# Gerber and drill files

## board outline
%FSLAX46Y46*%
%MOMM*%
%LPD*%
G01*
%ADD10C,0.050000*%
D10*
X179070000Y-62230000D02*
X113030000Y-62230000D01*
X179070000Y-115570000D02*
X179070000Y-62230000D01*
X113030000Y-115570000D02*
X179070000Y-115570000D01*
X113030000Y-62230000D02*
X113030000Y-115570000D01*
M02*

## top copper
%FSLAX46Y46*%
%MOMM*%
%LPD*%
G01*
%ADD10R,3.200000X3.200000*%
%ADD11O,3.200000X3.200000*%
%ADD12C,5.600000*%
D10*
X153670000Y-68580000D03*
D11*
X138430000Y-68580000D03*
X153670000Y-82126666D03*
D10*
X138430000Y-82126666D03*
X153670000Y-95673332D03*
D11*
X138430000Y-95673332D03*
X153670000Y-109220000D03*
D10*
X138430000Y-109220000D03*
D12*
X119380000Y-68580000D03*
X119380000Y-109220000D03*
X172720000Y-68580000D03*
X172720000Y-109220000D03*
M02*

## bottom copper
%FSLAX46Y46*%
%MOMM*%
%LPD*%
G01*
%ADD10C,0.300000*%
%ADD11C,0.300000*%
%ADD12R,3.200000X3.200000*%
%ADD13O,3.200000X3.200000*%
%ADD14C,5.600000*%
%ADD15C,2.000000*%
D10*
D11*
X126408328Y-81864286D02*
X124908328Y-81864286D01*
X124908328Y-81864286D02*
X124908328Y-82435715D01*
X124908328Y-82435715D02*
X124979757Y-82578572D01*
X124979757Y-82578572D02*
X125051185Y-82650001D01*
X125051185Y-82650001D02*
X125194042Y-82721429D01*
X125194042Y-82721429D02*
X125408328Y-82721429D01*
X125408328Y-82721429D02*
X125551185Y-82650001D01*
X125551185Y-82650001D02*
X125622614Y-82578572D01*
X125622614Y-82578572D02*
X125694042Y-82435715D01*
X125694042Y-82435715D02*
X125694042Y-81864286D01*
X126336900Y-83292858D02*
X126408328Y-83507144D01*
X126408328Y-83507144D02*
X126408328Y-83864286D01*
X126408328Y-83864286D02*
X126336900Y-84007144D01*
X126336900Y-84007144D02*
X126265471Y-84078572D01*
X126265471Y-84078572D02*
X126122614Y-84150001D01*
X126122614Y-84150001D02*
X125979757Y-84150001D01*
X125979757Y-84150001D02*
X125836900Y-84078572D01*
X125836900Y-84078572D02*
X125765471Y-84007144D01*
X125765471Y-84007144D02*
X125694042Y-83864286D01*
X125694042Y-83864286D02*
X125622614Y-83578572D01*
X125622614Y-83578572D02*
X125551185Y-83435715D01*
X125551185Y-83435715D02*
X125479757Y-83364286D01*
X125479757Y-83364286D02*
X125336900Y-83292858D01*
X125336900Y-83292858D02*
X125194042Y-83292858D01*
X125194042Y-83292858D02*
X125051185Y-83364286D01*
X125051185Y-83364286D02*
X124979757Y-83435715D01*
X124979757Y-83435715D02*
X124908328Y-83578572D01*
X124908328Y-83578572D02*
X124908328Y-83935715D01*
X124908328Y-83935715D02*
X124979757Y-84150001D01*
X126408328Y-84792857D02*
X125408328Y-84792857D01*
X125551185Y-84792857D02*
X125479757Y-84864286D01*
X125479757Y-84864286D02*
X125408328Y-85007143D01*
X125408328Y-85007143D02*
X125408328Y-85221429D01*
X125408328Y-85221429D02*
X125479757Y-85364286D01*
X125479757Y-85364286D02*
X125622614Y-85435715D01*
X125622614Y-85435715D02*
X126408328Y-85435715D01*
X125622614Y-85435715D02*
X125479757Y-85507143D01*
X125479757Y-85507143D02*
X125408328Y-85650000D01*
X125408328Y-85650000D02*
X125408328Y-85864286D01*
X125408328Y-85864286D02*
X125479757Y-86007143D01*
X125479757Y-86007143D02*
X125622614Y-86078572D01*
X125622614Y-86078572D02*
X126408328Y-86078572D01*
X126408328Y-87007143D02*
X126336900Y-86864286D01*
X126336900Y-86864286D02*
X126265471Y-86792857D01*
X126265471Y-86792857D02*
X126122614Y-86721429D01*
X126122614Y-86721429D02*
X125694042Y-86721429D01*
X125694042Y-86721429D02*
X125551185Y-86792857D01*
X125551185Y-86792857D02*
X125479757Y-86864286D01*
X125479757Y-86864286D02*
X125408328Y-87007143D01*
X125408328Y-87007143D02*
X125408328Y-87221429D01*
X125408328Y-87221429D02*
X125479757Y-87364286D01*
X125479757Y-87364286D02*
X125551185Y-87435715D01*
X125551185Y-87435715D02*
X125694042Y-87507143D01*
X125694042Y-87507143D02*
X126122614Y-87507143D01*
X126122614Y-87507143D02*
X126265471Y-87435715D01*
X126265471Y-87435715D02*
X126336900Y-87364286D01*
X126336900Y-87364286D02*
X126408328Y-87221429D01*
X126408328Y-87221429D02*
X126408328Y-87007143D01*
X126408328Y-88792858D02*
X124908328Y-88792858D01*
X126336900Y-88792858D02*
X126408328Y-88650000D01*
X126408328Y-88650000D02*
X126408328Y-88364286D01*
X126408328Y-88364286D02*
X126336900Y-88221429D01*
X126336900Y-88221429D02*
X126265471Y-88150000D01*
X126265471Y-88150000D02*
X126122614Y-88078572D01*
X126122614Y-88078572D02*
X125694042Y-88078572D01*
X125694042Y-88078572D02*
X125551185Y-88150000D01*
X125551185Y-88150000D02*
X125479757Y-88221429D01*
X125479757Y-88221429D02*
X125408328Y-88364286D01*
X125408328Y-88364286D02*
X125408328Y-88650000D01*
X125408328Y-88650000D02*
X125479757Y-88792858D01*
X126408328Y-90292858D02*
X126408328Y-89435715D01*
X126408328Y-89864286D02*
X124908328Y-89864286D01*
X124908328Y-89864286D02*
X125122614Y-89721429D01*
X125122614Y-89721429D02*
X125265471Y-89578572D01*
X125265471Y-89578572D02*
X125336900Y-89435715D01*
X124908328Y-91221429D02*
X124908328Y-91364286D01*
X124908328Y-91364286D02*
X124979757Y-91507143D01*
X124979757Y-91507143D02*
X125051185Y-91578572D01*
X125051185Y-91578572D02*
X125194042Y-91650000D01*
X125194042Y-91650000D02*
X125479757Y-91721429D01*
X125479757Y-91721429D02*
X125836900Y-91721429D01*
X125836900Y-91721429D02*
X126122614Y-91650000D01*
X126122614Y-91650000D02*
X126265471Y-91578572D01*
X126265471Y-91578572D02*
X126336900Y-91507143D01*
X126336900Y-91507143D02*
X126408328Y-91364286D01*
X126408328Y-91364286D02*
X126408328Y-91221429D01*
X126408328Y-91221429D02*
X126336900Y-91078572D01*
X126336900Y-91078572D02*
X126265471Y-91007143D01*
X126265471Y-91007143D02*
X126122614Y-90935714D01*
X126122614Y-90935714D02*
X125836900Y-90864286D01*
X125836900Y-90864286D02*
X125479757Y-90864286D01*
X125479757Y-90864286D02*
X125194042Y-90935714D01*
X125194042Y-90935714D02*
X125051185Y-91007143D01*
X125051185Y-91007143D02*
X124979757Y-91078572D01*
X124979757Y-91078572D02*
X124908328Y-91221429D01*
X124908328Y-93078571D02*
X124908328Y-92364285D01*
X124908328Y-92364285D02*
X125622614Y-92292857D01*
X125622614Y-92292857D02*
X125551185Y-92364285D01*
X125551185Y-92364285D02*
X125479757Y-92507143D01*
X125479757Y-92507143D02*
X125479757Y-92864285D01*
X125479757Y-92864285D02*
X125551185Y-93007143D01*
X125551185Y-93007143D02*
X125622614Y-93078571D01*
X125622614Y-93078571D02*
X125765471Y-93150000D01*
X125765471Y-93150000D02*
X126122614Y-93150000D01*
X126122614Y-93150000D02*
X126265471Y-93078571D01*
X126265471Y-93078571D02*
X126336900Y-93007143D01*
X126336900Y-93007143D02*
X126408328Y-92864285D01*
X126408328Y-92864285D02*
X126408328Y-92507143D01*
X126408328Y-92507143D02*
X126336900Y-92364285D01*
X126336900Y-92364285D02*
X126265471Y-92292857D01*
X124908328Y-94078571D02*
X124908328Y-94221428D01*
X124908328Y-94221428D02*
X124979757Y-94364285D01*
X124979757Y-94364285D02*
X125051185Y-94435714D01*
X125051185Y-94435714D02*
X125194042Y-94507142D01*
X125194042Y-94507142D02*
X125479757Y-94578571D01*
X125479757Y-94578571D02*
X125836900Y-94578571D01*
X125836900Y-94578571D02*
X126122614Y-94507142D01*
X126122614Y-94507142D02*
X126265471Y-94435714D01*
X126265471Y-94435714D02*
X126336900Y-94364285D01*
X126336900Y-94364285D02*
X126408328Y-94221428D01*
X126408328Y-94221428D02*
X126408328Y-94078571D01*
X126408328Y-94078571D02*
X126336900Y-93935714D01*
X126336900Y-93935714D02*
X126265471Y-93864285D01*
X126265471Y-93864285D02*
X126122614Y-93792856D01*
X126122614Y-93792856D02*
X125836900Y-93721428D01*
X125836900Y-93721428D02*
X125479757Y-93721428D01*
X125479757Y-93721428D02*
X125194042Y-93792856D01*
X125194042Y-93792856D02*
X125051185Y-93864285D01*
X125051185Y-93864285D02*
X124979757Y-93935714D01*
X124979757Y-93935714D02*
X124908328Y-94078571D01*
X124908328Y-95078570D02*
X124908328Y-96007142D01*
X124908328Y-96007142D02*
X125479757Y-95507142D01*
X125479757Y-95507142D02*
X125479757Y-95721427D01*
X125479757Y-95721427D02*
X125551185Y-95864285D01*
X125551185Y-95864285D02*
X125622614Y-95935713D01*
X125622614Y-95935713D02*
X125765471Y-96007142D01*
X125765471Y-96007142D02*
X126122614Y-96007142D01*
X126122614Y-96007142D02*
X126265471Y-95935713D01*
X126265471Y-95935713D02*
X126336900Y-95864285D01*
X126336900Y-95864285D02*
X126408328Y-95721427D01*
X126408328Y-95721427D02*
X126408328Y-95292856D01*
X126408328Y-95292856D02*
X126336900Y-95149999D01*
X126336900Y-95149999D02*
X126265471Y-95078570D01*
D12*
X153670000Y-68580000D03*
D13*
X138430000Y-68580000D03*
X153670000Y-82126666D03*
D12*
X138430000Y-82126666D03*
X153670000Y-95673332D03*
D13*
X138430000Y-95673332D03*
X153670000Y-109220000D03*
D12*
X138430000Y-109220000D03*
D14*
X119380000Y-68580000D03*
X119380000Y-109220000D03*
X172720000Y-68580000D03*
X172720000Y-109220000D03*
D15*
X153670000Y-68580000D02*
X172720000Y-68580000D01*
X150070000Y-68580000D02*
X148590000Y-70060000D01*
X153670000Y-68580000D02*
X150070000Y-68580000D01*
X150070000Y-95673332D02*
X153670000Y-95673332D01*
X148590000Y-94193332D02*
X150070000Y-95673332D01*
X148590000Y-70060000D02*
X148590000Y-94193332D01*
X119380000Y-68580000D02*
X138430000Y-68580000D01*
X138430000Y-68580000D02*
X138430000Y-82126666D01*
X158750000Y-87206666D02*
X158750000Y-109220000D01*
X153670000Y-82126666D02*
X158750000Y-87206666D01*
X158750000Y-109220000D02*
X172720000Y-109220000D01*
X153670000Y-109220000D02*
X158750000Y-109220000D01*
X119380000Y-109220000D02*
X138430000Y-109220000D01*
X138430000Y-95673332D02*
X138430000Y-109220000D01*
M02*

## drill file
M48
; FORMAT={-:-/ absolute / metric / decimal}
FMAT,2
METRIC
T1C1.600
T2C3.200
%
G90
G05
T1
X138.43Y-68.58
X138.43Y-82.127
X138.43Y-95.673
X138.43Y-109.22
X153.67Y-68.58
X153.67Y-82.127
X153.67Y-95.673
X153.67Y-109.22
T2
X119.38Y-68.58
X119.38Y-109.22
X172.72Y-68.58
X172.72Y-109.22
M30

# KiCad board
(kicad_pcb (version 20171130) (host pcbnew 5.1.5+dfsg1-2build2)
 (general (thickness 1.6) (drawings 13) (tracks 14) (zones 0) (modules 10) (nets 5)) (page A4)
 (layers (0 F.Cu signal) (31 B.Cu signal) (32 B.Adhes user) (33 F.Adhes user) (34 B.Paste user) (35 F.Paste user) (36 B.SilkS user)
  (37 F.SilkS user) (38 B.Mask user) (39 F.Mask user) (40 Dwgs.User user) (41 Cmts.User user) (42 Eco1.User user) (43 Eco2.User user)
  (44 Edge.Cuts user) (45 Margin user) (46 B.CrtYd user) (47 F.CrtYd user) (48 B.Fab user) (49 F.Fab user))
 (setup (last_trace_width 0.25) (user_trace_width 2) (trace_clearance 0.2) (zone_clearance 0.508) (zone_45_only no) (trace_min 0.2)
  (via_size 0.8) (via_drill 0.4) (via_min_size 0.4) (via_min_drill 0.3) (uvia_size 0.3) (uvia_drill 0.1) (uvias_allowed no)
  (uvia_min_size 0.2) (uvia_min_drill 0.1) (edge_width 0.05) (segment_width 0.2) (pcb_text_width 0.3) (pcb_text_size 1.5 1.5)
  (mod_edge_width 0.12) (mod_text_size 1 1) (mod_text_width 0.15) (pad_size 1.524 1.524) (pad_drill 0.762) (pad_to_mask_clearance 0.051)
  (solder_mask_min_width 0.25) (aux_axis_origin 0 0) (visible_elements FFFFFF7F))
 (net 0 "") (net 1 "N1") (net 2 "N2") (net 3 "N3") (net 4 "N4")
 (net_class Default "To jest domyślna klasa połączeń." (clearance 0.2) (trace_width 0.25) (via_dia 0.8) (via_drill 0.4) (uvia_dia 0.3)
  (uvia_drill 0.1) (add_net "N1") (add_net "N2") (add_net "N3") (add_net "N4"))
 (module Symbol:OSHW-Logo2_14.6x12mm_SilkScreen (layer F.Cu) (at 168.91 87.63)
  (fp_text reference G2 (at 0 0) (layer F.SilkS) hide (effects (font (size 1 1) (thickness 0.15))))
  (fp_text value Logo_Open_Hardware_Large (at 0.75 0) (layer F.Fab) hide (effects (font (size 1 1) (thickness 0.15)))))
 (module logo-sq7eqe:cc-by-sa (layer F.Cu) (at 125.73 87.63)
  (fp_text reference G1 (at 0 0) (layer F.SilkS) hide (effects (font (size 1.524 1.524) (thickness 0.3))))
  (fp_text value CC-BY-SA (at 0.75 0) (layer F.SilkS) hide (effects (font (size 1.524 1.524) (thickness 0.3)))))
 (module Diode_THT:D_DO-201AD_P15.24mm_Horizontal (layer F.Cu) (at 153.67 68.58 180)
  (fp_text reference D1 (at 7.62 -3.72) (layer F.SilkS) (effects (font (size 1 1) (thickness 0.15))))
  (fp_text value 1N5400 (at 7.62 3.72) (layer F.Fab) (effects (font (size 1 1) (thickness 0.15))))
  (pad 1 thru_hole rect (at 0 0 180) (size 3.2 3.2) (drill 1.6) (layers *.Cu *.Mask) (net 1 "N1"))
  (pad 2 thru_hole oval (at 15.24 0 180) (size 3.2 3.2) (drill 1.6) (layers *.Cu *.Mask) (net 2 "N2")))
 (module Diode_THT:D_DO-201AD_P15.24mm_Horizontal (layer F.Cu) (at 138.43 82.126666)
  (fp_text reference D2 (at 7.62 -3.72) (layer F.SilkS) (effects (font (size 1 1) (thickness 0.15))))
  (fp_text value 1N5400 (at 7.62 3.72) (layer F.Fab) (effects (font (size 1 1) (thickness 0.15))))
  (pad 2 thru_hole oval (at 15.24 0) (size 3.2 3.2) (drill 1.6) (layers *.Cu *.Mask) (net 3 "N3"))
  (pad 1 thru_hole rect (at 0 0) (size 3.2 3.2) (drill 1.6) (layers *.Cu *.Mask) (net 2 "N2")))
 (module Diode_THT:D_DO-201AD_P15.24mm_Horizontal (layer F.Cu) (at 153.67 95.673332 180)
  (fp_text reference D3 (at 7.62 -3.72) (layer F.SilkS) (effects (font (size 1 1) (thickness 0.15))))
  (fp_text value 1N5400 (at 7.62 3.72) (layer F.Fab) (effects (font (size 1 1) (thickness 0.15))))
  (pad 1 thru_hole rect (at 0 0 180) (size 3.2 3.2) (drill 1.6) (layers *.Cu *.Mask) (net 1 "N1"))
  (pad 2 thru_hole oval (at 15.24 0 180) (size 3.2 3.2) (drill 1.6) (layers *.Cu *.Mask) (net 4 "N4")))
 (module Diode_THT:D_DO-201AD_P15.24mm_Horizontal (layer F.Cu) (at 138.43 109.22)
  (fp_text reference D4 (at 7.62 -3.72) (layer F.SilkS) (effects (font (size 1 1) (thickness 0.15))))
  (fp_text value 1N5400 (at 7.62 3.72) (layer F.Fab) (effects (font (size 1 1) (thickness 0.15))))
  (pad 2 thru_hole oval (at 15.24 0) (size 3.2 3.2) (drill 1.6) (layers *.Cu *.Mask) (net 3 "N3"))
  (pad 1 thru_hole rect (at 0 0) (size 3.2 3.2) (drill 1.6) (layers *.Cu *.Mask) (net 4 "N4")))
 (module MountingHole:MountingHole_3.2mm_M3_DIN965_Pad (layer F.Cu) (at 119.38 68.58)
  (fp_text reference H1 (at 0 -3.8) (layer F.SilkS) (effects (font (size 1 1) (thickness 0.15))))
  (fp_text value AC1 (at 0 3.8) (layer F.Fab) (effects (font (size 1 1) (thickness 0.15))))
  (pad 1 thru_hole circle (at 0 0) (size 5.6 5.6) (drill 3.2) (layers *.Cu *.Mask) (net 2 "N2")))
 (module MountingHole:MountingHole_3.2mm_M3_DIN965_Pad (layer F.Cu) (at 119.38 109.22)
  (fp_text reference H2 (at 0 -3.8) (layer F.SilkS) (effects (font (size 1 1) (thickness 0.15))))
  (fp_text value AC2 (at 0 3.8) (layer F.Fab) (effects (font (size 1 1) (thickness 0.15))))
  (pad 1 thru_hole circle (at 0 0) (size 5.6 5.6) (drill 3.2) (layers *.Cu *.Mask) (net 4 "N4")))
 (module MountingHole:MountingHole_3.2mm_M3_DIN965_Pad (layer F.Cu) (at 172.72 68.58)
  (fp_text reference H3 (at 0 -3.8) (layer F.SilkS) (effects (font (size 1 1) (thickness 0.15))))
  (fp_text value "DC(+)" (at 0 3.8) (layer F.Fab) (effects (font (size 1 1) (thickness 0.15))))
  (pad 1 thru_hole circle (at 0 0) (size 5.6 5.6) (drill 3.2) (layers *.Cu *.Mask) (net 1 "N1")))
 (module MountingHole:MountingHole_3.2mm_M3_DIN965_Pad (layer F.Cu) (at 172.72 109.22)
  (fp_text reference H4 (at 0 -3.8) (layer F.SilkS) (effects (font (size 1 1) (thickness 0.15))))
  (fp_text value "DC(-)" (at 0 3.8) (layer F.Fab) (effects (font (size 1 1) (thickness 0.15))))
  (pad 1 thru_hole circle (at 0 0) (size 5.6 5.6) (drill 3.2) (layers *.Cu *.Mask) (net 3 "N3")))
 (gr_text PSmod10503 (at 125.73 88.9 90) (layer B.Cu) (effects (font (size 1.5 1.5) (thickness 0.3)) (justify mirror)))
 (gr_line (start 179.07 62.23) (end 113.03 62.23) (layer Edge.Cuts) (width 0.05))
 (gr_line (start 179.07 115.57) (end 179.07 62.23) (layer Edge.Cuts) (width 0.05))
 (gr_line (start 113.03 115.57) (end 179.07 115.57) (layer Edge.Cuts) (width 0.05))
 (gr_line (start 113.03 62.23) (end 113.03 115.57) (layer Edge.Cuts) (width 0.05))
 (segment (start 153.67 68.58) (end 172.72 68.58) (width 2) (layer B.Cu) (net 1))
 (segment (start 150.07 68.58) (end 148.59 70.06) (width 2) (layer B.Cu) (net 1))
 (segment (start 153.67 68.58) (end 150.07 68.58) (width 2) (layer B.Cu) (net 1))
 (segment (start 150.07 95.673332) (end 153.67 95.673332) (width 2) (layer B.Cu) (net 1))
 (segment (start 148.59 94.193332) (end 150.07 95.673332) (width 2) (layer B.Cu) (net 1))
 (segment (start 148.59 70.06) (end 148.59 94.193332) (width 2) (layer B.Cu) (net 1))
 (segment (start 119.38 68.58) (end 138.43 68.58) (width 2) (layer B.Cu) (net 2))
 (segment (start 138.43 68.58) (end 138.43 82.126666) (width 2) (layer B.Cu) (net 2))
 (segment (start 158.75 87.206666) (end 158.75 109.22) (width 2) (layer B.Cu) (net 3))
 (segment (start 153.67 82.126666) (end 158.75 87.206666) (width 2) (layer B.Cu) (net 3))
 (segment (start 158.75 109.22) (end 172.72 109.22) (width 2) (layer B.Cu) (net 3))
 (segment (start 153.67 109.22) (end 158.75 109.22) (width 2) (layer B.Cu) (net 3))
 (segment (start 119.38 109.22) (end 138.43 109.22) (width 2) (layer B.Cu) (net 4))
 (segment (start 138.43 95.673332) (end 138.43 109.22) (width 2) (layer B.Cu) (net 4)))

